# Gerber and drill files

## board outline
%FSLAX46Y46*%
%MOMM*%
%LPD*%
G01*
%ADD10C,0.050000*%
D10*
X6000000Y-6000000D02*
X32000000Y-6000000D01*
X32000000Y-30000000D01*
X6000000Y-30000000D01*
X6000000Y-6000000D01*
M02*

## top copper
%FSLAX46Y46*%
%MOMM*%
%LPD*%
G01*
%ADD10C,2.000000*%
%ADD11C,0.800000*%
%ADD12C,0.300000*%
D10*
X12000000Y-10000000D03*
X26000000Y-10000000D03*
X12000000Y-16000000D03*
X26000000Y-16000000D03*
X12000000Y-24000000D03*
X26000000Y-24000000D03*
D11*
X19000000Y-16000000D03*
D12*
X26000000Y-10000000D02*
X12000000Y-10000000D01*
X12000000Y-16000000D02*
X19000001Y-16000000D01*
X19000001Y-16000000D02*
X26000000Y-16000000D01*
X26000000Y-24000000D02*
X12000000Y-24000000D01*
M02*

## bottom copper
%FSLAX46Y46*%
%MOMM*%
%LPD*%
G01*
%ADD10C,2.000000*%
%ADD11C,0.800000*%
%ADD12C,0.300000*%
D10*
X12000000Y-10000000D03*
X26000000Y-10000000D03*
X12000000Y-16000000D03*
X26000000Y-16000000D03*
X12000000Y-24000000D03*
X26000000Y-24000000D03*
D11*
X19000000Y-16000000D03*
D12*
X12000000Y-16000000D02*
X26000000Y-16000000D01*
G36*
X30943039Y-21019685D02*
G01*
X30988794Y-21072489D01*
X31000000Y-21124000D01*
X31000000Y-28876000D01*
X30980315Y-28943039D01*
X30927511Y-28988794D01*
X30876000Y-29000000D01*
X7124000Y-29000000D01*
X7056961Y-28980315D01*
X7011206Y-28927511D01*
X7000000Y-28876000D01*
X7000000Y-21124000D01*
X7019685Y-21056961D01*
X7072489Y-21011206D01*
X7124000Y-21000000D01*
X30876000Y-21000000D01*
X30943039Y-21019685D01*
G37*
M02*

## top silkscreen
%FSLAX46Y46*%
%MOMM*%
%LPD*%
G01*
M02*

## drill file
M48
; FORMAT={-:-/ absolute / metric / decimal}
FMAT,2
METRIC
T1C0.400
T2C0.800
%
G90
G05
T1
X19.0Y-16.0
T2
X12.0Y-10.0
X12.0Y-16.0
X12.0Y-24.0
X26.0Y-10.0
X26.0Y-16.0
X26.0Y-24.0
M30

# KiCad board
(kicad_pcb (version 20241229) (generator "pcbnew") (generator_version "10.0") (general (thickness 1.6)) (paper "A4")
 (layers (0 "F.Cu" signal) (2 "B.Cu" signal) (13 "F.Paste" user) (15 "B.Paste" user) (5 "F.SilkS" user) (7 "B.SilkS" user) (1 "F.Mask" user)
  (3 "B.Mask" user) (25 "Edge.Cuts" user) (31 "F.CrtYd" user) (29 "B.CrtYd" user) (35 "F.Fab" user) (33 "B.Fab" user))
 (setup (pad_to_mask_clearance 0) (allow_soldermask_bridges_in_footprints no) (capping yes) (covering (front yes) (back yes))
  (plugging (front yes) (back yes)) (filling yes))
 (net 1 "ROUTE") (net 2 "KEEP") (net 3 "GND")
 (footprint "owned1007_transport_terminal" (layer "F.Cu") (at 12 10)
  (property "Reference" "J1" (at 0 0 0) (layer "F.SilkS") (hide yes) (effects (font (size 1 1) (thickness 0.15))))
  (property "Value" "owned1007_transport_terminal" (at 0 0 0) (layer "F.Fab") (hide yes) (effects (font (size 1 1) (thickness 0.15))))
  (pad "1" thru_hole circle (at 0 0) (size 2 2) (drill 0.8) (layers "*.Cu" "*.Mask") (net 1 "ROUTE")))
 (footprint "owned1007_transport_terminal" (layer "F.Cu") (at 26 10)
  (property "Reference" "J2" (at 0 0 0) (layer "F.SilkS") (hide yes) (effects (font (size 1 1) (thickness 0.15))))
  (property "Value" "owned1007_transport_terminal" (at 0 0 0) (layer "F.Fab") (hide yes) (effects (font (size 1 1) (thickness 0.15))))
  (pad "1" thru_hole circle (at 0 0) (size 2 2) (drill 0.8) (layers "*.Cu" "*.Mask") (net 1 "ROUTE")))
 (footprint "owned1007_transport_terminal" (layer "F.Cu") (at 12 16)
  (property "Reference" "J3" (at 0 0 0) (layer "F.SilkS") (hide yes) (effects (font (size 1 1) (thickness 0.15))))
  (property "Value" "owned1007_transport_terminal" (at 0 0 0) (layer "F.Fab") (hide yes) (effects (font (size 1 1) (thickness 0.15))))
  (pad "1" thru_hole circle (at 0 0) (size 2 2) (drill 0.8) (layers "*.Cu" "*.Mask") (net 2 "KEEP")))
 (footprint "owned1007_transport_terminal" (layer "F.Cu") (at 26 16)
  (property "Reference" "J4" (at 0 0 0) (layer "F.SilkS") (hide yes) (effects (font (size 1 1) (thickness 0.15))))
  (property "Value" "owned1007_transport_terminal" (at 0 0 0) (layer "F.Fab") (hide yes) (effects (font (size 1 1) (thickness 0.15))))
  (pad "1" thru_hole circle (at 0 0) (size 2 2) (drill 0.8) (layers "*.Cu" "*.Mask") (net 2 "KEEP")))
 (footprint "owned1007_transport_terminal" (layer "F.Cu") (at 12 24)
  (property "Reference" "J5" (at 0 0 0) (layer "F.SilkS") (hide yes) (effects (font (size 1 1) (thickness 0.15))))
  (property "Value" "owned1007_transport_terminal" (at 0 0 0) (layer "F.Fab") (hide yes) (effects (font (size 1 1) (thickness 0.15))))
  (pad "1" thru_hole circle (at 0 0) (size 2 2) (drill 0.8) (layers "*.Cu" "*.Mask") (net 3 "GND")))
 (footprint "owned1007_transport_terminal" (layer "F.Cu") (at 26 24)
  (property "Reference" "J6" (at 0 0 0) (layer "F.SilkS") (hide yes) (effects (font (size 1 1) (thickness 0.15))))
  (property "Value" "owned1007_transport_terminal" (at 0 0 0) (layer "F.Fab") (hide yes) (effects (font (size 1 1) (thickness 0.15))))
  (pad "1" thru_hole circle (at 0 0) (size 2 2) (drill 0.8) (layers "*.Cu" "*.Mask") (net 3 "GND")))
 (gr_rect (start 6 6) (end 32 30) (stroke (width 0.05) (type default)) (fill none) (layer "Edge.Cuts"))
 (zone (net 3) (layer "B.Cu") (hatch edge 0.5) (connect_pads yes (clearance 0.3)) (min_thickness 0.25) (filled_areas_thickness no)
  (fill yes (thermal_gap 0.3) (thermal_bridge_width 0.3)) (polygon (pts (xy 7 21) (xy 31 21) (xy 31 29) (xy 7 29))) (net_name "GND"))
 (segment (start 26 10) (end 12 10) (width 0.3) (layer "F.Cu") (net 1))
 (segment (start 12 16) (end 19.000001 16) (width 0.3) (layer "F.Cu") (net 2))
 (segment (start 19.000001 16) (end 26 16) (width 0.3) (layer "F.Cu") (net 2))
 (via (at 19 16) (size 0.8) (drill 0.4) (layers "F.Cu" "B.Cu") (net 2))
 (segment (start 12 16) (end 26 16) (width 0.3) (layer "B.Cu") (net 2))
 (segment (start 26 24) (end 12 24) (width 0.3) (layer "F.Cu") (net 3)))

